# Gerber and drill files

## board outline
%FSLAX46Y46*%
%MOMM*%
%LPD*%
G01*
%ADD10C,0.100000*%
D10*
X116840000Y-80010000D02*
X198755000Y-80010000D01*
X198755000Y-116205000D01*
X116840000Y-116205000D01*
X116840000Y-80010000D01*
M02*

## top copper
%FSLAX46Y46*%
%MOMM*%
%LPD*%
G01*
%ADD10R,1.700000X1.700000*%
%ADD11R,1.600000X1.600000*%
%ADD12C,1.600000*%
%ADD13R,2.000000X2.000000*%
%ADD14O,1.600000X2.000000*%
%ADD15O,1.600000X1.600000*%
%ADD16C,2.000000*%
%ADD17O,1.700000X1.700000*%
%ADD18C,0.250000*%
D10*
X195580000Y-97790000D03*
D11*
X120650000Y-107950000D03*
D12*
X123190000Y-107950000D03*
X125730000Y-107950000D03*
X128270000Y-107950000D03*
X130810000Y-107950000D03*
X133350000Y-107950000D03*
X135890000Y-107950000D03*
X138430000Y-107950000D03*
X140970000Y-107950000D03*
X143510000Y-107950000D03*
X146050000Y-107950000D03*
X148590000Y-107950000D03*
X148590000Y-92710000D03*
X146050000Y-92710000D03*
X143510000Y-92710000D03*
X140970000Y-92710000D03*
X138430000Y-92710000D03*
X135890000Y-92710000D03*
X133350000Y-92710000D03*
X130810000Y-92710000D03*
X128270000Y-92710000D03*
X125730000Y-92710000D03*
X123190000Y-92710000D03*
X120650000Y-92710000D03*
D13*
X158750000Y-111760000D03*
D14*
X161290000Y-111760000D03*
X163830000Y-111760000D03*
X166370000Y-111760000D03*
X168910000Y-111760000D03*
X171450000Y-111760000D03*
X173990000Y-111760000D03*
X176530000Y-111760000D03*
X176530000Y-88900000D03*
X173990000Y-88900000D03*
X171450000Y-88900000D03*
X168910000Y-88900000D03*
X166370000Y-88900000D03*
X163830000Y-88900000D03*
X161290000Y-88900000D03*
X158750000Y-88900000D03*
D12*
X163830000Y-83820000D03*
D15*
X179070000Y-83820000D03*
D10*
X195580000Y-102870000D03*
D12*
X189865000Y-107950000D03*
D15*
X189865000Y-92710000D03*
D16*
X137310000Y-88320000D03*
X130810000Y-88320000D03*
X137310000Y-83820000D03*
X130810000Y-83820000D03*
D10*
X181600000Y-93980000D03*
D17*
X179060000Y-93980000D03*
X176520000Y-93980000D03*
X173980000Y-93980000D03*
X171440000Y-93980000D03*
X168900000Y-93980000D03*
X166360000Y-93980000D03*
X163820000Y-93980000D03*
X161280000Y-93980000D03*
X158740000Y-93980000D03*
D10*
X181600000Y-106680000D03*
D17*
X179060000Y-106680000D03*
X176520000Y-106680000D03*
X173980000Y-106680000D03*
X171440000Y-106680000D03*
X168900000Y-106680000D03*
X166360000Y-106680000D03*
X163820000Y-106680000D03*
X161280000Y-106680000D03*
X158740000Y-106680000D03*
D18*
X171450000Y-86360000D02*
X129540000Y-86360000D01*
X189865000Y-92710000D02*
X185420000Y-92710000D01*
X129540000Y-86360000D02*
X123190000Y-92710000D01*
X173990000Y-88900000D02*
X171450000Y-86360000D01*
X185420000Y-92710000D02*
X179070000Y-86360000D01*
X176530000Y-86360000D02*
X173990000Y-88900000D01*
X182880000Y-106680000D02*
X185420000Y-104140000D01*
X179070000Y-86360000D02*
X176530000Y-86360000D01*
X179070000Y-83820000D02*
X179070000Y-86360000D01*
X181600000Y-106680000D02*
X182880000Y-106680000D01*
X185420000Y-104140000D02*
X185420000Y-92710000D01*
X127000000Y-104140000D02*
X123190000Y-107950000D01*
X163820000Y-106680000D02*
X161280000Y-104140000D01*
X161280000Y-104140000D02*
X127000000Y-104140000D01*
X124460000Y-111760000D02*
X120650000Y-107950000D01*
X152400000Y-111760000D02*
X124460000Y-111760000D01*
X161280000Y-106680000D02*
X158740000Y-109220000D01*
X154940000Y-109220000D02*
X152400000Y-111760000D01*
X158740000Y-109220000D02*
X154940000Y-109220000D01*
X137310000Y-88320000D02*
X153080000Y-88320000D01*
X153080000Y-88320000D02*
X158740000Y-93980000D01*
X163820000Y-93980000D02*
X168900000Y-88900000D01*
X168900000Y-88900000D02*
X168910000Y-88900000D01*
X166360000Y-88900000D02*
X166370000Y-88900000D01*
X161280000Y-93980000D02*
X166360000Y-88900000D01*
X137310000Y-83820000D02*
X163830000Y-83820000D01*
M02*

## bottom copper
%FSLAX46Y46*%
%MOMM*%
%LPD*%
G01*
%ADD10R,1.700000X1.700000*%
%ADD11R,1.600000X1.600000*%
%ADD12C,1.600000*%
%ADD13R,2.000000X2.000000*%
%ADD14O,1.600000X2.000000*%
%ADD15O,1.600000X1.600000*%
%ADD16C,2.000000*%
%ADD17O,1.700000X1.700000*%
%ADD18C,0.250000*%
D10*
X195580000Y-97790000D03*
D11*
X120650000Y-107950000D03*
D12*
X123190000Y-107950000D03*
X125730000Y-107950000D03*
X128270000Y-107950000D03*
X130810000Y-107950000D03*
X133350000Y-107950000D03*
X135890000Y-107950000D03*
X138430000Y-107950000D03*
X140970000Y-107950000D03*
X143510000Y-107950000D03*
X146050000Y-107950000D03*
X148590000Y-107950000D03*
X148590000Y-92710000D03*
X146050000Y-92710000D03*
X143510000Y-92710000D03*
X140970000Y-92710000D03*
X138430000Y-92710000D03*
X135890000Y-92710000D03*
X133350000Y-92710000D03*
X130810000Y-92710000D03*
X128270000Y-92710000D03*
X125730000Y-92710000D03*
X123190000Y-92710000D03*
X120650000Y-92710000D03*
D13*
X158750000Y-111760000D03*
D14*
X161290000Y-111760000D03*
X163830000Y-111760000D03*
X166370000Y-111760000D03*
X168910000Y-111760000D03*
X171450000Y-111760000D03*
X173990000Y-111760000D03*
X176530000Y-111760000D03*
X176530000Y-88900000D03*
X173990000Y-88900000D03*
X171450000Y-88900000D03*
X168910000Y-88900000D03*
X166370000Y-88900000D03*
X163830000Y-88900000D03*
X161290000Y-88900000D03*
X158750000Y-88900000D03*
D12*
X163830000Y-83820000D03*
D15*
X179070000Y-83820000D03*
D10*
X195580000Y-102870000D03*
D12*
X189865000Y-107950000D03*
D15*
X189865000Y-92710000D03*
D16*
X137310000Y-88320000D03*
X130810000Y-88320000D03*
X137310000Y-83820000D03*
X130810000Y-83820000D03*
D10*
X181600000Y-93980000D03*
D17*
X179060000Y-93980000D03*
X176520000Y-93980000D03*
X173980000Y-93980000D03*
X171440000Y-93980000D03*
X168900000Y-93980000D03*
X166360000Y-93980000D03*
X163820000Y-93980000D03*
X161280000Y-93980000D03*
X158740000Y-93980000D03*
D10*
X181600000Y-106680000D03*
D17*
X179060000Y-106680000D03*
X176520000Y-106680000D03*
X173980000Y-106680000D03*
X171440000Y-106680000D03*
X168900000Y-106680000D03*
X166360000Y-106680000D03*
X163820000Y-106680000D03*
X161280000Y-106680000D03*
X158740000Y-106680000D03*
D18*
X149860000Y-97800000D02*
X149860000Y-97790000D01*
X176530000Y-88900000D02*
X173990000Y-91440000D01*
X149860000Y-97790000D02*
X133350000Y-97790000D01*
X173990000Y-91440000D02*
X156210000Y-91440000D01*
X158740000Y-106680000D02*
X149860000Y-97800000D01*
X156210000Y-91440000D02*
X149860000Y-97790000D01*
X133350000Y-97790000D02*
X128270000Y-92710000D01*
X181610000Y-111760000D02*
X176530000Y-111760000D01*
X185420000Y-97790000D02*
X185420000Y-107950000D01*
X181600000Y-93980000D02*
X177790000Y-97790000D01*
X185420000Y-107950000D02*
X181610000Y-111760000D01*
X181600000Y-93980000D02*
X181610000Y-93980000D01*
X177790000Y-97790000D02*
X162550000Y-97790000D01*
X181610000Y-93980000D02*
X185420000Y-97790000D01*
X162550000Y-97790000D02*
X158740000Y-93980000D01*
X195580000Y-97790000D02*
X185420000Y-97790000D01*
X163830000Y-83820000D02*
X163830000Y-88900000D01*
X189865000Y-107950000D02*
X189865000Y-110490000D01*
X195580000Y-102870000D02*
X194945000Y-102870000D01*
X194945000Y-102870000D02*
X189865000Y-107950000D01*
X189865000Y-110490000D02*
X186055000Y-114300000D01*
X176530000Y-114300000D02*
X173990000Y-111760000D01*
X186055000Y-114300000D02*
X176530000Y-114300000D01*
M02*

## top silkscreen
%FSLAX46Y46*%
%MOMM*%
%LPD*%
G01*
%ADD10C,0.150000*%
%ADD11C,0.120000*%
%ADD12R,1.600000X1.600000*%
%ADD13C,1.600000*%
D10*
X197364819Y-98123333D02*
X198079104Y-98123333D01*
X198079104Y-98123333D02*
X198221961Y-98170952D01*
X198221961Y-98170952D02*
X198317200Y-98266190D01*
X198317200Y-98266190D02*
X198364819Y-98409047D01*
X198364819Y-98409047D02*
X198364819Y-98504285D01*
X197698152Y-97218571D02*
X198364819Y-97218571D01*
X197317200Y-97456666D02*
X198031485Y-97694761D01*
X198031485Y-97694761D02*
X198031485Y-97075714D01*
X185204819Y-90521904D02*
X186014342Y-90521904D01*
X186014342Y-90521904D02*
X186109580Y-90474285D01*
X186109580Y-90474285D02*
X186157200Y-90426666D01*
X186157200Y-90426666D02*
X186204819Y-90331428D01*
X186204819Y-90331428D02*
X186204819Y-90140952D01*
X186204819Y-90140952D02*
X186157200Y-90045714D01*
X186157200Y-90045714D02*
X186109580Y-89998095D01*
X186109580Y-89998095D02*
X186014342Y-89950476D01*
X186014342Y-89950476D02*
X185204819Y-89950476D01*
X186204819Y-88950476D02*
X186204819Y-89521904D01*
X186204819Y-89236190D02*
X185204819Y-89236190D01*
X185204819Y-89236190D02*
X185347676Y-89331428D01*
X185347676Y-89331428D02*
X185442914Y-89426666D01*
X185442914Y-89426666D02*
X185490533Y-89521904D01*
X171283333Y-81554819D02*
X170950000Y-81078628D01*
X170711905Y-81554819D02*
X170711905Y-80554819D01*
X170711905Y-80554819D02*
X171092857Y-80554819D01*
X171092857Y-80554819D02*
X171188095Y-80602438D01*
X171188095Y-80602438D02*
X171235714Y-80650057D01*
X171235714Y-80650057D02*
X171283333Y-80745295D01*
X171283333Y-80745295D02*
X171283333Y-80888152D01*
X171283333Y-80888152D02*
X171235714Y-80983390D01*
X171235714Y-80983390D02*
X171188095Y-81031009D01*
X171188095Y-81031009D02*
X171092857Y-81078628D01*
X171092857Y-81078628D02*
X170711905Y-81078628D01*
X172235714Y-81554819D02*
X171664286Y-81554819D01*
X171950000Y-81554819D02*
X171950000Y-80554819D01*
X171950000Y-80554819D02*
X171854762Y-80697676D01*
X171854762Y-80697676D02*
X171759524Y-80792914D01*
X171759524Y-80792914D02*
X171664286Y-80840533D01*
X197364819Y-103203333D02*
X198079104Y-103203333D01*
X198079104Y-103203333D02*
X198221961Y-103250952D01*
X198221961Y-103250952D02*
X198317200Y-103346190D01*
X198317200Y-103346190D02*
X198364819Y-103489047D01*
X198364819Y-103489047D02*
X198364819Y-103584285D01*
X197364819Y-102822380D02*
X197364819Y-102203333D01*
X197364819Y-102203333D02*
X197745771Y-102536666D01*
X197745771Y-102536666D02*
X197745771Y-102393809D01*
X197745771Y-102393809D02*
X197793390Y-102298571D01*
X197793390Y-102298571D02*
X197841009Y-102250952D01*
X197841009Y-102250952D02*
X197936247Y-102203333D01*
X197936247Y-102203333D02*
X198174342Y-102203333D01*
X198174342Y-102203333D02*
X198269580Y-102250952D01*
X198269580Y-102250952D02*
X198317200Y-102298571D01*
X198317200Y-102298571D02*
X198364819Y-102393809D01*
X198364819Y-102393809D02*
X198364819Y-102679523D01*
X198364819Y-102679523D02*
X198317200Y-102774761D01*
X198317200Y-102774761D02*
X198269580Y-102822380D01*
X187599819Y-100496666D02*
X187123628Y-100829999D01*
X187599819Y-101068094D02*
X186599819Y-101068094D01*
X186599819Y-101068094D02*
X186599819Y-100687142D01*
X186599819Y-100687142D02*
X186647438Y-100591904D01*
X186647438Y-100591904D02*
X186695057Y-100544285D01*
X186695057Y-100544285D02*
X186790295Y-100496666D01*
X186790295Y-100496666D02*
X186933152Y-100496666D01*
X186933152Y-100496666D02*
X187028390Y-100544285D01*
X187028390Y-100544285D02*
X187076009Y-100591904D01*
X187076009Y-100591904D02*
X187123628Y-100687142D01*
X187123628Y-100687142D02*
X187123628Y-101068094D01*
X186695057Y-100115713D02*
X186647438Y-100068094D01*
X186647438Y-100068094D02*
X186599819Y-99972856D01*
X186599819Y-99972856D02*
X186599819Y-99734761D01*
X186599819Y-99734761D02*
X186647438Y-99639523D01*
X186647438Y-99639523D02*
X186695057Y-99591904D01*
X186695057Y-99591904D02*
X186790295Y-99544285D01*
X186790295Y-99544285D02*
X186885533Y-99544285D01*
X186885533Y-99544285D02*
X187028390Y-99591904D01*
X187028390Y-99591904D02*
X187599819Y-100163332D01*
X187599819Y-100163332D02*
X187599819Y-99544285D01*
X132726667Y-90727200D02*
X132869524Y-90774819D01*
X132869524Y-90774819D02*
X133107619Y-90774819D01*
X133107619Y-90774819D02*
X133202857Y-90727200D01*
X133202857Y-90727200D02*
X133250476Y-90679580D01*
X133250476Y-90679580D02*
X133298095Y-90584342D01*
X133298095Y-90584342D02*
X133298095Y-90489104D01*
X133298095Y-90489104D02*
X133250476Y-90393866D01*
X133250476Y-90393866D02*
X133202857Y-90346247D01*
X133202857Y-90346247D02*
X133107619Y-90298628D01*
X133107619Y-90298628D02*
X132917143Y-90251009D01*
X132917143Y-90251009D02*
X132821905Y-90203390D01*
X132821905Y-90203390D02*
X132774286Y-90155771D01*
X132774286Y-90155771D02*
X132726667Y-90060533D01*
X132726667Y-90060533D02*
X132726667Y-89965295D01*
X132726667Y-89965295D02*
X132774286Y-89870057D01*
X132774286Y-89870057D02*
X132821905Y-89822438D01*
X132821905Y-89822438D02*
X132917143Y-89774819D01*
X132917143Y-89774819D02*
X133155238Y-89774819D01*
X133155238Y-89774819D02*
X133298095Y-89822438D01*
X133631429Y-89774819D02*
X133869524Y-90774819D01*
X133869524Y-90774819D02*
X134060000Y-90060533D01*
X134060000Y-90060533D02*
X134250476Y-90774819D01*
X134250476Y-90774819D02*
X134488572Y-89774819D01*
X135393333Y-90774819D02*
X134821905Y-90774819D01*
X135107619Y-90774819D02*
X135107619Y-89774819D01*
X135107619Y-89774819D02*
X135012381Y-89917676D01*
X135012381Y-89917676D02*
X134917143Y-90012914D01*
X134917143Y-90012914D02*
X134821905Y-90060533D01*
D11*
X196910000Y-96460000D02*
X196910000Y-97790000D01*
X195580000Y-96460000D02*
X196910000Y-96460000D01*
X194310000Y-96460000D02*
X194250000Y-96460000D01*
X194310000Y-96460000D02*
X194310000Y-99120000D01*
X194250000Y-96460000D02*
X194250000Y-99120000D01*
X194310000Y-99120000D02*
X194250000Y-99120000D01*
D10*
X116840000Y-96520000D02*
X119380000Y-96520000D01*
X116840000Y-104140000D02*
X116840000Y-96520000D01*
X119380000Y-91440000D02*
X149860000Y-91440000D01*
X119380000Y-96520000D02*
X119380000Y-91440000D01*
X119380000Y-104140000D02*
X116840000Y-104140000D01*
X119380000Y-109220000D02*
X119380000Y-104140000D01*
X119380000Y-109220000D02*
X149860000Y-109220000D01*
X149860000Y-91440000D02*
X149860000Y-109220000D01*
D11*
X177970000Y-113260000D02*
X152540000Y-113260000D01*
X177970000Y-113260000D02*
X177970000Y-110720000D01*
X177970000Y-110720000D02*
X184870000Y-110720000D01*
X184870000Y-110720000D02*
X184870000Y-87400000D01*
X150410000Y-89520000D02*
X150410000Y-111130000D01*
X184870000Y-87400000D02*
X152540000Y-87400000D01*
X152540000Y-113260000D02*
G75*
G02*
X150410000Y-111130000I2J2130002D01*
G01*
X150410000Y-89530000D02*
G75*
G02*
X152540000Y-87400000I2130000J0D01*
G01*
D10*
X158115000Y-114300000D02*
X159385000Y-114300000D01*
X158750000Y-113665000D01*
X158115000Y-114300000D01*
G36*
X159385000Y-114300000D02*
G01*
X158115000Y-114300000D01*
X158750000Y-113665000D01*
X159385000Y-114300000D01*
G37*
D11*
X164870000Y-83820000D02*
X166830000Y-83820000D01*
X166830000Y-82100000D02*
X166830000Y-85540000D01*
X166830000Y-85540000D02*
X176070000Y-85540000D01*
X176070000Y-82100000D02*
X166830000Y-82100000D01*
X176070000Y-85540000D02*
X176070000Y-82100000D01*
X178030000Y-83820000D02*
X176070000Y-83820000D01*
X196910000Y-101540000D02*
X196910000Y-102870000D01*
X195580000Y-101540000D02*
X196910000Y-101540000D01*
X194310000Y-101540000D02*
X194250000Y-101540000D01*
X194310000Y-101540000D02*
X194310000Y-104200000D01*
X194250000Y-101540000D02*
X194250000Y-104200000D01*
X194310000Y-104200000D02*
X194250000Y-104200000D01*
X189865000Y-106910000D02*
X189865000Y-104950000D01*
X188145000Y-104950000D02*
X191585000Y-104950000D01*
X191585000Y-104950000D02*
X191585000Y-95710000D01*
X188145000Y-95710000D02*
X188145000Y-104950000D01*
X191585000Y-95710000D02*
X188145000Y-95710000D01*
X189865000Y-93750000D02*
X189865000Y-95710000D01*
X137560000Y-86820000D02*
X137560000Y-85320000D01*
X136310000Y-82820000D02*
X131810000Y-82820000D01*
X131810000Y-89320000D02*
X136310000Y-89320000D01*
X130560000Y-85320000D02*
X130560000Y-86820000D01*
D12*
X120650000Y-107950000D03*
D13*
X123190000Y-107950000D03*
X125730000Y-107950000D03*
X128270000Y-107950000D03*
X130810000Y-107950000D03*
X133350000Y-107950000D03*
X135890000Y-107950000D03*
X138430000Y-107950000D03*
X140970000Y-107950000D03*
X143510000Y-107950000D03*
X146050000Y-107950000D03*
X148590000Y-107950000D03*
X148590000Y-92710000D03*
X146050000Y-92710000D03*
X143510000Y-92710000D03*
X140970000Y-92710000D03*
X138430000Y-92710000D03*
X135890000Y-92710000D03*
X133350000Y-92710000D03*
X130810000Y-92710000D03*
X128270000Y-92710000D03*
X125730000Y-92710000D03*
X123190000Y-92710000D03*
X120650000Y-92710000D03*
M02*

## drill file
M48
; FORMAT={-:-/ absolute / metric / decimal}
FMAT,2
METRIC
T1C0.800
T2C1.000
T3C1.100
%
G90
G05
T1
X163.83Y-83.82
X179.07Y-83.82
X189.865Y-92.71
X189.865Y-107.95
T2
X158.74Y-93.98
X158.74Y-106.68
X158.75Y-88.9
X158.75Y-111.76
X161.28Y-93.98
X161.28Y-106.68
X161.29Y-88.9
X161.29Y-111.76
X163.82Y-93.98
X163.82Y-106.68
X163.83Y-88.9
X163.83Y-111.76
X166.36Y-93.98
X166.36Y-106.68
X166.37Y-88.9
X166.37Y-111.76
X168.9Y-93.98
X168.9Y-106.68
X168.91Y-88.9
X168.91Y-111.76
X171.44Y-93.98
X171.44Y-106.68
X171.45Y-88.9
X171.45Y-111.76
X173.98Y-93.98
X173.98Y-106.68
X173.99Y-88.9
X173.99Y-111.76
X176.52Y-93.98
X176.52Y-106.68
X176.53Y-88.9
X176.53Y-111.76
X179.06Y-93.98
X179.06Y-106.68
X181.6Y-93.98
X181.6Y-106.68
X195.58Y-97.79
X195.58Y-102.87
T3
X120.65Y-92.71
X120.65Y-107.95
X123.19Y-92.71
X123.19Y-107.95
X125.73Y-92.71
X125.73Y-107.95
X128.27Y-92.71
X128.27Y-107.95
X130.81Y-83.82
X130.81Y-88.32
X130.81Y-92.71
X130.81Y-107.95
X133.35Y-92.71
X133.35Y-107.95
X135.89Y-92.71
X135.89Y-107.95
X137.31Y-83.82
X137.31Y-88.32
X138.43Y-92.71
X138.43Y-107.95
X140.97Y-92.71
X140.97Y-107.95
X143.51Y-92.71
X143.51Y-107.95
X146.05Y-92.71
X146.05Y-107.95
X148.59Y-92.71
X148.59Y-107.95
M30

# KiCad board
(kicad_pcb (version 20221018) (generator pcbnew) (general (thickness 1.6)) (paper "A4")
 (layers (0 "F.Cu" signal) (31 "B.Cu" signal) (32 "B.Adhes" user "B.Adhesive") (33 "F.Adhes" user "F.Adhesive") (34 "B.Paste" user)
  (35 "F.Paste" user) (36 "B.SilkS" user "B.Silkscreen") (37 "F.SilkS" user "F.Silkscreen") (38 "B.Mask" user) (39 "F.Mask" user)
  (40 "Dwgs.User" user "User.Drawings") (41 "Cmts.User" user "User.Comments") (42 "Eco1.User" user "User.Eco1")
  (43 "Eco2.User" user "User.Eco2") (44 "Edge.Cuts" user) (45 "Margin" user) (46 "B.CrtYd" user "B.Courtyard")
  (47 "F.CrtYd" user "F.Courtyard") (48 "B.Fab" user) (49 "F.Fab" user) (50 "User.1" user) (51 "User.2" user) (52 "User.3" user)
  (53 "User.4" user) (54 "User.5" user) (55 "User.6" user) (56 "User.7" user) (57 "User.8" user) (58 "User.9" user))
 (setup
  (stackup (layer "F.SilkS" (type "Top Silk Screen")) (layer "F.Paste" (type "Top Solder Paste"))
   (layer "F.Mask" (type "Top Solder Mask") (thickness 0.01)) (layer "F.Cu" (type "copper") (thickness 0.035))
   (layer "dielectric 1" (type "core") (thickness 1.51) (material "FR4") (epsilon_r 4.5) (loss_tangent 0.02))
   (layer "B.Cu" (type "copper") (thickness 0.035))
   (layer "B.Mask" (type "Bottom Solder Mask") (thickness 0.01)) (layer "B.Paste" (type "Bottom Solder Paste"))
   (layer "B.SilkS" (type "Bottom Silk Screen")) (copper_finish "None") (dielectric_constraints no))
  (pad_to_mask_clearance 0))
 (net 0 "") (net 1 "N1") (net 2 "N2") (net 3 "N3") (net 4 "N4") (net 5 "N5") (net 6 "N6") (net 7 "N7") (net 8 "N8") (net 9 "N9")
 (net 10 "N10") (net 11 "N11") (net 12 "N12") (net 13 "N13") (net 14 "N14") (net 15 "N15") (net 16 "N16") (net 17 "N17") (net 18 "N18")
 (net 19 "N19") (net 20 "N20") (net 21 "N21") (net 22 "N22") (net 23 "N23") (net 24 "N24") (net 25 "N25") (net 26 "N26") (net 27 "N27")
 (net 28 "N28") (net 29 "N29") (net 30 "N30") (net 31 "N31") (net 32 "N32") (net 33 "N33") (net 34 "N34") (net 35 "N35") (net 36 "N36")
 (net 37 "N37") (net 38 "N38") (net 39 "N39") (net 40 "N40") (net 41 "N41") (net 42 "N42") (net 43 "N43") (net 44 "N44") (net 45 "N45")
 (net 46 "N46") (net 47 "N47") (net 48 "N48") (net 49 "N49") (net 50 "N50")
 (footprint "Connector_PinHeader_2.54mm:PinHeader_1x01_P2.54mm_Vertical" (layer "F.Cu") (at 195.58 97.79 -90)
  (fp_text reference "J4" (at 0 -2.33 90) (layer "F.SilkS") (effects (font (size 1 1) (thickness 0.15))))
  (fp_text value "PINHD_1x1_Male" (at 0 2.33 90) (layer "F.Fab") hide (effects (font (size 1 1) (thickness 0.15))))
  (fp_line (start -1.33 -1.33) (end 0 -1.33) (stroke (width 0.12) (type solid)) (layer "F.SilkS"))
  (fp_line (start -1.33 0) (end -1.33 -1.33) (stroke (width 0.12) (type solid)) (layer "F.SilkS"))
  (fp_line (start -1.33 1.27) (end -1.33 1.33) (stroke (width 0.12) (type solid)) (layer "F.SilkS"))
  (fp_line (start -1.33 1.27) (end 1.33 1.27) (stroke (width 0.12) (type solid)) (layer "F.SilkS"))
  (fp_line (start -1.33 1.33) (end 1.33 1.33) (stroke (width 0.12) (type solid)) (layer "F.SilkS"))
  (fp_line (start 1.33 1.27) (end 1.33 1.33) (stroke (width 0.12) (type solid)) (layer "F.SilkS"))
  (pad "1" thru_hole rect (at 0 0 270) (size 1.7 1.7) (drill 1) (layers "*.Cu" "*.Mask") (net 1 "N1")))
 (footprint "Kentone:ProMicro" (layer "F.Cu") (at 134.62 100.33)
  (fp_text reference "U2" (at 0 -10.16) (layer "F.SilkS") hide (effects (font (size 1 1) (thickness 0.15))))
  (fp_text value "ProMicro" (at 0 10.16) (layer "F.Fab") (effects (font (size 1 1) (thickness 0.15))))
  (fp_line (start -17.78 -3.81) (end -15.24 -3.81) (stroke (width 0.15) (type solid)) (layer "F.SilkS"))
  (fp_line (start -17.78 3.81) (end -17.78 -3.81) (stroke (width 0.15) (type solid)) (layer "F.SilkS"))
  (fp_line (start -15.24 -8.89) (end 15.24 -8.89) (stroke (width 0.15) (type solid)) (layer "F.SilkS"))
  (fp_line (start -15.24 -3.81) (end -15.24 -8.89) (stroke (width 0.15) (type solid)) (layer "F.SilkS"))
  (fp_line (start -15.24 3.81) (end -17.78 3.81) (stroke (width 0.15) (type solid)) (layer "F.SilkS"))
  (fp_line (start -15.24 8.89) (end -15.24 3.81) (stroke (width 0.15) (type solid)) (layer "F.SilkS"))
  (fp_line (start -15.24 8.89) (end 15.24 8.89) (stroke (width 0.15) (type solid)) (layer "F.SilkS"))
  (fp_line (start 15.24 -8.89) (end 15.24 8.89) (stroke (width 0.15) (type solid)) (layer "F.SilkS"))
  (pad "1" thru_hole rect (at -13.97 7.62) (size 1.6 1.6) (drill 1.1) (layers "*.Cu" "*.Mask" "F.SilkS") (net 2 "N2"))
  (pad "2" thru_hole circle (at -11.43 7.62) (size 1.6 1.6) (drill 1.1) (layers "*.Cu" "*.Mask" "F.SilkS") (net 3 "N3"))
  (pad "3" thru_hole circle (at -8.89 7.62) (size 1.6 1.6) (drill 1.1) (layers "*.Cu" "*.Mask" "F.SilkS") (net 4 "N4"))
  (pad "4" thru_hole circle (at -6.35 7.62) (size 1.6 1.6) (drill 1.1) (layers "*.Cu" "*.Mask" "F.SilkS") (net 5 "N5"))
  (pad "5" thru_hole circle (at -3.81 7.62) (size 1.6 1.6) (drill 1.1) (layers "*.Cu" "*.Mask" "F.SilkS") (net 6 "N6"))
  (pad "6" thru_hole circle (at -1.27 7.62) (size 1.6 1.6) (drill 1.1) (layers "*.Cu" "*.Mask" "F.SilkS") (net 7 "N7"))
  (pad "7" thru_hole circle (at 1.27 7.62) (size 1.6 1.6) (drill 1.1) (layers "*.Cu" "*.Mask" "F.SilkS") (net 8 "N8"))
  (pad "8" thru_hole circle (at 3.81 7.62) (size 1.6 1.6) (drill 1.1) (layers "*.Cu" "*.Mask" "F.SilkS") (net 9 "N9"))
  (pad "9" thru_hole circle (at 6.35 7.62) (size 1.6 1.6) (drill 1.1) (layers "*.Cu" "*.Mask" "F.SilkS") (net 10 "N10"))
  (pad "10" thru_hole circle (at 8.89 7.62) (size 1.6 1.6) (drill 1.1) (layers "*.Cu" "*.Mask" "F.SilkS") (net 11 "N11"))
  (pad "11" thru_hole circle (at 11.43 7.62) (size 1.6 1.6) (drill 1.1) (layers "*.Cu" "*.Mask" "F.SilkS") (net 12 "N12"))
  (pad "12" thru_hole circle (at 13.97 7.62) (size 1.6 1.6) (drill 1.1) (layers "*.Cu" "*.Mask" "F.SilkS") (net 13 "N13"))
  (pad "13" thru_hole circle (at 13.97 -7.62) (size 1.6 1.6) (drill 1.1) (layers "*.Cu" "*.Mask" "F.SilkS") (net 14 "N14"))
  (pad "14" thru_hole circle (at 11.43 -7.62) (size 1.6 1.6) (drill 1.1) (layers "*.Cu" "*.Mask" "F.SilkS") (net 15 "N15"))
  (pad "15" thru_hole circle (at 8.89 -7.62) (size 1.6 1.6) (drill 1.1) (layers "*.Cu" "*.Mask" "F.SilkS") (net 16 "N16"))
  (pad "16" thru_hole circle (at 6.35 -7.62) (size 1.6 1.6) (drill 1.1) (layers "*.Cu" "*.Mask" "F.SilkS") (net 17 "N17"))
  (pad "17" thru_hole circle (at 3.81 -7.62) (size 1.6 1.6) (drill 1.1) (layers "*.Cu" "*.Mask" "F.SilkS") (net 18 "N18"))
  (pad "18" thru_hole circle (at 1.27 -7.62) (size 1.6 1.6) (drill 1.1) (layers "*.Cu" "*.Mask" "F.SilkS") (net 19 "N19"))
  (pad "19" thru_hole circle (at -1.27 -7.62) (size 1.6 1.6) (drill 1.1) (layers "*.Cu" "*.Mask" "F.SilkS") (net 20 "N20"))
  (pad "20" thru_hole circle (at -3.81 -7.62) (size 1.6 1.6) (drill 1.1) (layers "*.Cu" "*.Mask" "F.SilkS") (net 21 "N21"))
  (pad "21" thru_hole circle (at -6.35 -7.62) (size 1.6 1.6) (drill 1.1) (layers "*.Cu" "*.Mask" "F.SilkS") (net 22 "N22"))
  (pad "22" thru_hole circle (at -8.89 -7.62) (size 1.6 1.6) (drill 1.1) (layers "*.Cu" "*.Mask" "F.SilkS") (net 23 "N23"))
  (pad "23" thru_hole circle (at -11.43 -7.62) (size 1.6 1.6) (drill 1.1) (layers "*.Cu" "*.Mask" "F.SilkS") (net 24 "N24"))
  (pad "24" thru_hole circle (at -13.97 -7.62) (size 1.6 1.6) (drill 1.1) (layers "*.Cu" "*.Mask" "F.SilkS") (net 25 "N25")))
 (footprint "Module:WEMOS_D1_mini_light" (layer "F.Cu") (at 158.75 111.76 90)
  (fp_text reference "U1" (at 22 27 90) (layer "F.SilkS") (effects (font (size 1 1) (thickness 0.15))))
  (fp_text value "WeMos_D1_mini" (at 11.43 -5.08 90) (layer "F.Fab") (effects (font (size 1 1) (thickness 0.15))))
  (fp_line (start -1.5 19.22) (end -1.5 -6.21) (stroke (width 0.12) (type solid)) (layer "F.SilkS"))
  (fp_line (start -1.5 19.22) (end 1.04 19.22) (stroke (width 0.12) (type solid)) (layer "F.SilkS"))
  (fp_line (start 1.04 19.22) (end 1.04 26.12) (stroke (width 0.12) (type solid)) (layer "F.SilkS"))
  (fp_line (start 1.04 26.12) (end 24.36 26.12) (stroke (width 0.12) (type solid)) (layer "F.SilkS"))
  (fp_line (start 22.24 -8.34) (end 0.63 -8.34) (stroke (width 0.12) (type solid)) (layer "F.SilkS"))
  (fp_line (start 24.36 26.12) (end 24.36 -6.21) (stroke (width 0.12) (type solid)) (layer "F.SilkS"))
  (fp_arc (start -1.5 -6.21) (mid -0.876137 -7.716137) (end 0.63 -8.34) (stroke (width 0.12) (type solid)) (layer "F.SilkS"))
  (fp_arc (start 22.23 -8.34) (mid 23.736137 -7.716137) (end 24.36 -6.21) (stroke (width 0.12) (type solid)) (layer "F.SilkS"))
  (fp_poly (pts (xy -2.54 -0.635) (xy -2.54 0.635) (xy -1.905 0)) (stroke (width 0.15) (type solid)) (fill solid) (layer "F.SilkS"))
  (pad "1" thru_hole rect (at 0 0 90) (size 2 2) (drill 1) (layers "*.Cu" "*.Mask") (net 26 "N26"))
  (pad "2" thru_hole oval (at 0 2.54 90) (size 2 1.6) (drill 1) (layers "*.Cu" "*.Mask") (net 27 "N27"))
  (pad "3" thru_hole oval (at 0 5.08 90) (size 2 1.6) (drill 1) (layers "*.Cu" "*.Mask") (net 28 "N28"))
  (pad "4" thru_hole oval (at 0 7.62 90) (size 2 1.6) (drill 1) (layers "*.Cu" "*.Mask") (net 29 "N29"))
  (pad "5" thru_hole oval (at 0 10.16 90) (size 2 1.6) (drill 1) (layers "*.Cu" "*.Mask") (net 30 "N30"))
  (pad "6" thru_hole oval (at 0 12.7 90) (size 2 1.6) (drill 1) (layers "*.Cu" "*.Mask") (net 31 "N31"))
  (pad "7" thru_hole oval (at 0 15.24 90) (size 2 1.6) (drill 1) (layers "*.Cu" "*.Mask") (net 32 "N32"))
  (pad "8" thru_hole oval (at 0 17.78 90) (size 2 1.6) (drill 1) (layers "*.Cu" "*.Mask") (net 1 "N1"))
  (pad "9" thru_hole oval (at 22.86 17.78 90) (size 2 1.6) (drill 1) (layers "*.Cu" "*.Mask") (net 22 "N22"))
  (pad "10" thru_hole oval (at 22.86 15.24 90) (size 2 1.6) (drill 1) (layers "*.Cu" "*.Mask") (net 24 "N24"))
  (pad "11" thru_hole oval (at 22.86 12.7 90) (size 2 1.6) (drill 1) (layers "*.Cu" "*.Mask") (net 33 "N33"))
  (pad "12" thru_hole oval (at 22.86 10.16 90) (size 2 1.6) (drill 1) (layers "*.Cu" "*.Mask") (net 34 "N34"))
  (pad "13" thru_hole oval (at 22.86 7.62 90) (size 2 1.6) (drill 1) (layers "*.Cu" "*.Mask") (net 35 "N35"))
  (pad "14" thru_hole oval (at 22.86 5.08 90) (size 2 1.6) (drill 1) (layers "*.Cu" "*.Mask") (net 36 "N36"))
  (pad "15" thru_hole oval (at 22.86 2.54 90) (size 2 1.6) (drill 1) (layers "*.Cu" "*.Mask") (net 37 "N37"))
  (pad "16" thru_hole oval (at 22.86 0 90) (size 2 1.6) (drill 1) (layers "*.Cu" "*.Mask") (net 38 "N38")))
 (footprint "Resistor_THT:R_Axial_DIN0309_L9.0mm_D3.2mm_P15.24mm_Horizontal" (layer "F.Cu") (at 163.83 83.82)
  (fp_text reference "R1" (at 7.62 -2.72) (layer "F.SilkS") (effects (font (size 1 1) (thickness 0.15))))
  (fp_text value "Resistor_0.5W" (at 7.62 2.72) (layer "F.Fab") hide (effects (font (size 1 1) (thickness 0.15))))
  (fp_line (start 1.04 0) (end 3 0) (stroke (width 0.12) (type solid)) (layer "F.SilkS"))
  (fp_line (start 3 -1.72) (end 3 1.72) (stroke (width 0.12) (type solid)) (layer "F.SilkS"))
  (fp_line (start 3 1.72) (end 12.24 1.72) (stroke (width 0.12) (type solid)) (layer "F.SilkS"))
  (fp_line (start 12.24 -1.72) (end 3 -1.72) (stroke (width 0.12) (type solid)) (layer "F.SilkS"))
  (fp_line (start 12.24 1.72) (end 12.24 -1.72) (stroke (width 0.12) (type solid)) (layer "F.SilkS"))
  (fp_line (start 14.2 0) (end 12.24 0) (stroke (width 0.12) (type solid)) (layer "F.SilkS"))
  (pad "1" thru_hole circle (at 0 0) (size 1.6 1.6) (drill 0.8) (layers "*.Cu" "*.Mask") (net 36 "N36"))
  (pad "2" thru_hole oval (at 15.24 0) (size 1.6 1.6) (drill 0.8) (layers "*.Cu" "*.Mask") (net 24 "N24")))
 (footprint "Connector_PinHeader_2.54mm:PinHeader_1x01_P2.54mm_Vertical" (layer "F.Cu") (at 195.58 102.87 -90)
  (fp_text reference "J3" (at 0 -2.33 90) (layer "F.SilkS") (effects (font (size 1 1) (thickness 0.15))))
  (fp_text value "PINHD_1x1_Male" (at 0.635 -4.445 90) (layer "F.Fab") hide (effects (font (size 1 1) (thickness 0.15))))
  (fp_line (start -1.33 -1.33) (end 0 -1.33) (stroke (width 0.12) (type solid)) (layer "F.SilkS"))
  (fp_line (start -1.33 0) (end -1.33 -1.33) (stroke (width 0.12) (type solid)) (layer "F.SilkS"))
  (fp_line (start -1.33 1.27) (end -1.33 1.33) (stroke (width 0.12) (type solid)) (layer "F.SilkS"))
  (fp_line (start -1.33 1.27) (end 1.33 1.27) (stroke (width 0.12) (type solid)) (layer "F.SilkS"))
  (fp_line (start -1.33 1.33) (end 1.33 1.33) (stroke (width 0.12) (type solid)) (layer "F.SilkS"))
  (fp_line (start 1.33 1.27) (end 1.33 1.33) (stroke (width 0.12) (type solid)) (layer "F.SilkS"))
  (pad "1" thru_hole rect (at 0 0 270) (size 1.7 1.7) (drill 1) (layers "*.Cu" "*.Mask") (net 32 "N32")))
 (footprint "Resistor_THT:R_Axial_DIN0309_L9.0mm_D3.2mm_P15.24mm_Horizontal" (layer "F.Cu") (at 189.865 107.95 90)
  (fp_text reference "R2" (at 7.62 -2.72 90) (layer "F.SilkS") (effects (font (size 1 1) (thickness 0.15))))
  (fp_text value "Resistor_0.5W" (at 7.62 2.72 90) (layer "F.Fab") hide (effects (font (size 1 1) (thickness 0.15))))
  (fp_line (start 1.04 0) (end 3 0) (stroke (width 0.12) (type solid)) (layer "F.SilkS"))
  (fp_line (start 3 -1.72) (end 3 1.72) (stroke (width 0.12) (type solid)) (layer "F.SilkS"))
  (fp_line (start 3 1.72) (end 12.24 1.72) (stroke (width 0.12) (type solid)) (layer "F.SilkS"))
  (fp_line (start 12.24 -1.72) (end 3 -1.72) (stroke (width 0.12) (type solid)) (layer "F.SilkS"))
  (fp_line (start 12.24 1.72) (end 12.24 -1.72) (stroke (width 0.12) (type solid)) (layer "F.SilkS"))
  (fp_line (start 14.2 0) (end 12.24 0) (stroke (width 0.12) (type solid)) (layer "F.SilkS"))
  (pad "1" thru_hole circle (at 0 0 90) (size 1.6 1.6) (drill 0.8) (layers "*.Cu" "*.Mask") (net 32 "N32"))
  (pad "2" thru_hole oval (at 15.24 0 90) (size 1.6 1.6) (drill 0.8) (layers "*.Cu" "*.Mask") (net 24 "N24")))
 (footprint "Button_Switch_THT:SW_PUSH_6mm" (layer "F.Cu") (at 137.31 88.32 180)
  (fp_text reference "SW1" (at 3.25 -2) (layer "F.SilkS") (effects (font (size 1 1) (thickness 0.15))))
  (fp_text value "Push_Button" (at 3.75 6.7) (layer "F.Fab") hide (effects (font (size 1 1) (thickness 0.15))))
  (fp_line (start -0.25 1.5) (end -0.25 3) (stroke (width 0.12) (type solid)) (layer "F.SilkS"))
  (fp_line (start 1 5.5) (end 5.5 5.5) (stroke (width 0.12) (type solid)) (layer "F.SilkS"))
  (fp_line (start 5.5 -1) (end 1 -1) (stroke (width 0.12) (type solid)) (layer "F.SilkS"))
  (fp_line (start 6.75 3) (end 6.75 1.5) (stroke (width 0.12) (type solid)) (layer "F.SilkS"))
  (pad "1" thru_hole circle (at 0 0 270) (size 2 2) (drill 1.1) (layers "*.Cu" "*.Mask") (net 1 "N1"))
  (pad "1" thru_hole circle (at 6.5 0 270) (size 2 2) (drill 1.1) (layers "*.Cu" "*.Mask") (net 1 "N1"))
  (pad "2" thru_hole circle (at 0 4.5 270) (size 2 2) (drill 1.1) (layers "*.Cu" "*.Mask") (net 36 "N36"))
  (pad "2" thru_hole circle (at 6.5 4.5 270) (size 2 2) (drill 1.1) (layers "*.Cu" "*.Mask") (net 36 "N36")))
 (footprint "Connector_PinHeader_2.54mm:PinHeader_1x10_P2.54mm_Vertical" (layer "B.Cu") (at 181.6 93.98 90)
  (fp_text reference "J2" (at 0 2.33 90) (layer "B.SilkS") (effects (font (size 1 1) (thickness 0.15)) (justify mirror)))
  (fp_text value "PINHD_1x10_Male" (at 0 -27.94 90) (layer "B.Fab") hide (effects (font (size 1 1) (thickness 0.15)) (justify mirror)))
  (pad "1" thru_hole rect (at 0 0 90) (size 1.7 1.7) (drill 1) (layers "*.Cu" "*.Mask") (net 1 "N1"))
  (pad "2" thru_hole oval (at 0 -2.54 90) (size 1.7 1.7) (drill 1) (layers "*.Cu" "*.Mask") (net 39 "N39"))
  (pad "3" thru_hole oval (at 0 -5.08 90) (size 1.7 1.7) (drill 1) (layers "*.Cu" "*.Mask") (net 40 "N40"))
  (pad "4" thru_hole oval (at 0 -7.62 90) (size 1.7 1.7) (drill 1) (layers "*.Cu" "*.Mask") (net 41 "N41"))
  (pad "5" thru_hole oval (at 0 -10.16 90) (size 1.7 1.7) (drill 1) (layers "*.Cu" "*.Mask") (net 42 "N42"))
  (pad "6" thru_hole oval (at 0 -12.7 90) (size 1.7 1.7) (drill 1) (layers "*.Cu" "*.Mask") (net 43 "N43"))
  (pad "7" thru_hole oval (at 0 -15.24 90) (size 1.7 1.7) (drill 1) (layers "*.Cu" "*.Mask") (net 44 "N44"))
  (pad "8" thru_hole oval (at 0 -17.78 90) (size 1.7 1.7) (drill 1) (layers "*.Cu" "*.Mask") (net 34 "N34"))
  (pad "9" thru_hole oval (at 0 -20.32 90) (size 1.7 1.7) (drill 1) (layers "*.Cu" "*.Mask") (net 35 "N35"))
  (pad "10" thru_hole oval (at 0 -22.86 90) (size 1.7 1.7) (drill 1) (layers "*.Cu" "*.Mask") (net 1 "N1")))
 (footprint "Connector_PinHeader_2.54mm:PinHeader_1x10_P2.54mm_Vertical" (layer "B.Cu") (at 181.6 106.68 90)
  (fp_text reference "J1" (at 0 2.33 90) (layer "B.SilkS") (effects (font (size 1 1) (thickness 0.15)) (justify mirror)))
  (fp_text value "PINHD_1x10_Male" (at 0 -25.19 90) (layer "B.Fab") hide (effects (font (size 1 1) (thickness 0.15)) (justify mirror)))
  (pad "1" thru_hole rect (at 0 0 90) (size 1.7 1.7) (drill 1) (layers "*.Cu" "*.Mask") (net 24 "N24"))
  (pad "2" thru_hole oval (at 0 -2.54 90) (size 1.7 1.7) (drill 1) (layers "*.Cu" "*.Mask") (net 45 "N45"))
  (pad "3" thru_hole oval (at 0 -5.08 90) (size 1.7 1.7) (drill 1) (layers "*.Cu" "*.Mask") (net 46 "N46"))
  (pad "4" thru_hole oval (at 0 -7.62 90) (size 1.7 1.7) (drill 1) (layers "*.Cu" "*.Mask") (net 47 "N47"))
  (pad "5" thru_hole oval (at 0 -10.16 90) (size 1.7 1.7) (drill 1) (layers "*.Cu" "*.Mask") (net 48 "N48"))
  (pad "6" thru_hole oval (at 0 -12.7 90) (size 1.7 1.7) (drill 1) (layers "*.Cu" "*.Mask") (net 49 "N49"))
  (pad "7" thru_hole oval (at 0 -15.24 90) (size 1.7 1.7) (drill 1) (layers "*.Cu" "*.Mask") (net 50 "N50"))
  (pad "8" thru_hole oval (at 0 -17.78 90) (size 1.7 1.7) (drill 1) (layers "*.Cu" "*.Mask") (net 3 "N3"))
  (pad "9" thru_hole oval (at 0 -20.32 90) (size 1.7 1.7) (drill 1) (layers "*.Cu" "*.Mask") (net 2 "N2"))
  (pad "10" thru_hole oval (at 0 -22.86 90) (size 1.7 1.7) (drill 1) (layers "*.Cu" "*.Mask") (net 22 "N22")))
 (gr_rect (start 116.84 80.01) (end 198.755 116.205) (stroke (width 0.1) (type default)) (fill none) (layer "Edge.Cuts"))
 (segment (start 171.45 86.36) (end 129.54 86.36) (width 0.25) (layer "F.Cu") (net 24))
 (segment (start 189.865 92.71) (end 185.42 92.71) (width 0.25) (layer "F.Cu") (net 24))
 (segment (start 129.54 86.36) (end 123.19 92.71) (width 0.25) (layer "F.Cu") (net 24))
 (segment (start 173.99 88.9) (end 171.45 86.36) (width 0.25) (layer "F.Cu") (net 24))
 (segment (start 185.42 92.71) (end 179.07 86.36) (width 0.25) (layer "F.Cu") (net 24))
 (segment (start 176.53 86.36) (end 173.99 88.9) (width 0.25) (layer "F.Cu") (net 24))
 (segment (start 182.88 106.68) (end 185.42 104.14) (width 0.25) (layer "F.Cu") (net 24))
 (segment (start 179.07 86.36) (end 176.53 86.36) (width 0.25) (layer "F.Cu") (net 24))
 (segment (start 179.07 83.82) (end 179.07 86.36) (width 0.25) (layer "F.Cu") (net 24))
 (segment (start 181.6 106.68) (end 182.88 106.68) (width 0.25) (layer "F.Cu") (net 24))
 (segment (start 185.42 104.14) (end 185.42 92.71) (width 0.25) (layer "F.Cu") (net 24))
 (segment (start 127 104.14) (end 123.19 107.95) (width 0.25) (layer "F.Cu") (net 3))
 (segment (start 163.82 106.68) (end 161.28 104.14) (width 0.25) (layer "F.Cu") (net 3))
 (segment (start 161.28 104.14) (end 127 104.14) (width 0.25) (layer "F.Cu") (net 3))
 (segment (start 124.46 111.76) (end 120.65 107.95) (width 0.25) (layer "F.Cu") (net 2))
 (segment (start 152.4 111.76) (end 124.46 111.76) (width 0.25) (layer "F.Cu") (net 2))
 (segment (start 161.28 106.68) (end 158.74 109.22) (width 0.25) (layer "F.Cu") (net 2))
 (segment (start 154.94 109.22) (end 152.4 111.76) (width 0.25) (layer "F.Cu") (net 2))
 (segment (start 158.74 109.22) (end 154.94 109.22) (width 0.25) (layer "F.Cu") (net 2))
 (segment (start 149.86 97.8) (end 149.86 97.79) (width 0.25) (layer "B.Cu") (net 22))
 (segment (start 176.53 88.9) (end 173.99 91.44) (width 0.25) (layer "B.Cu") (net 22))
 (segment (start 149.86 97.79) (end 133.35 97.79) (width 0.25) (layer "B.Cu") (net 22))
 (segment (start 173.99 91.44) (end 156.21 91.44) (width 0.25) (layer "B.Cu") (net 22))
 (segment (start 158.74 106.68) (end 149.86 97.8) (width 0.25) (layer "B.Cu") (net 22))
 (segment (start 156.21 91.44) (end 149.86 97.79) (width 0.25) (layer "B.Cu") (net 22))
 (segment (start 133.35 97.79) (end 128.27 92.71) (width 0.25) (layer "B.Cu") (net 22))
 (segment (start 137.31 88.32) (end 153.08 88.32) (width 0.25) (layer "F.Cu") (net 1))
 (segment (start 153.08 88.32) (end 158.74 93.98) (width 0.25) (layer "F.Cu") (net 1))
 (segment (start 181.61 111.76) (end 176.53 111.76) (width 0.25) (layer "B.Cu") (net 1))
 (segment (start 185.42 97.79) (end 185.42 107.95) (width 0.25) (layer "B.Cu") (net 1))
 (segment (start 181.6 93.98) (end 177.79 97.79) (width 0.25) (layer "B.Cu") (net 1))
 (segment (start 185.42 107.95) (end 181.61 111.76) (width 0.25) (layer "B.Cu") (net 1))
 (segment (start 181.6 93.98) (end 181.61 93.98) (width 0.25) (layer "B.Cu") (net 1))
 (segment (start 177.79 97.79) (end 162.55 97.79) (width 0.25) (layer "B.Cu") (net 1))
 (segment (start 181.61 93.98) (end 185.42 97.79) (width 0.25) (layer "B.Cu") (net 1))
 (segment (start 162.55 97.79) (end 158.74 93.98) (width 0.25) (layer "B.Cu") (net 1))
 (segment (start 195.58 97.79) (end 185.42 97.79) (width 0.25) (layer "B.Cu") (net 1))
 (segment (start 163.82 93.98) (end 168.9 88.9) (width 0.25) (layer "F.Cu") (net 34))
 (segment (start 168.9 88.9) (end 168.91 88.9) (width 0.25) (layer "F.Cu") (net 34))
 (segment (start 166.36 88.9) (end 166.37 88.9) (width 0.25) (layer "F.Cu") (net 35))
 (segment (start 161.28 93.98) (end 166.36 88.9) (width 0.25) (layer "F.Cu") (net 35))
 (segment (start 137.31 83.82) (end 163.83 83.82) (width 0.25) (layer "F.Cu") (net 36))
 (segment (start 163.83 83.82) (end 163.83 88.9) (width 0.25) (layer "B.Cu") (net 36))
 (segment (start 189.865 107.95) (end 189.865 110.49) (width 0.25) (layer "B.Cu") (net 32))
 (segment (start 195.58 102.87) (end 194.945 102.87) (width 0.25) (layer "B.Cu") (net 32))
 (segment (start 194.945 102.87) (end 189.865 107.95) (width 0.25) (layer "B.Cu") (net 32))
 (segment (start 189.865 110.49) (end 186.055 114.3) (width 0.25) (layer "B.Cu") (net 32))
 (segment (start 176.53 114.3) (end 173.99 111.76) (width 0.25) (layer "B.Cu") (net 32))
 (segment (start 186.055 114.3) (end 176.53 114.3) (width 0.25) (layer "B.Cu") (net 32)))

